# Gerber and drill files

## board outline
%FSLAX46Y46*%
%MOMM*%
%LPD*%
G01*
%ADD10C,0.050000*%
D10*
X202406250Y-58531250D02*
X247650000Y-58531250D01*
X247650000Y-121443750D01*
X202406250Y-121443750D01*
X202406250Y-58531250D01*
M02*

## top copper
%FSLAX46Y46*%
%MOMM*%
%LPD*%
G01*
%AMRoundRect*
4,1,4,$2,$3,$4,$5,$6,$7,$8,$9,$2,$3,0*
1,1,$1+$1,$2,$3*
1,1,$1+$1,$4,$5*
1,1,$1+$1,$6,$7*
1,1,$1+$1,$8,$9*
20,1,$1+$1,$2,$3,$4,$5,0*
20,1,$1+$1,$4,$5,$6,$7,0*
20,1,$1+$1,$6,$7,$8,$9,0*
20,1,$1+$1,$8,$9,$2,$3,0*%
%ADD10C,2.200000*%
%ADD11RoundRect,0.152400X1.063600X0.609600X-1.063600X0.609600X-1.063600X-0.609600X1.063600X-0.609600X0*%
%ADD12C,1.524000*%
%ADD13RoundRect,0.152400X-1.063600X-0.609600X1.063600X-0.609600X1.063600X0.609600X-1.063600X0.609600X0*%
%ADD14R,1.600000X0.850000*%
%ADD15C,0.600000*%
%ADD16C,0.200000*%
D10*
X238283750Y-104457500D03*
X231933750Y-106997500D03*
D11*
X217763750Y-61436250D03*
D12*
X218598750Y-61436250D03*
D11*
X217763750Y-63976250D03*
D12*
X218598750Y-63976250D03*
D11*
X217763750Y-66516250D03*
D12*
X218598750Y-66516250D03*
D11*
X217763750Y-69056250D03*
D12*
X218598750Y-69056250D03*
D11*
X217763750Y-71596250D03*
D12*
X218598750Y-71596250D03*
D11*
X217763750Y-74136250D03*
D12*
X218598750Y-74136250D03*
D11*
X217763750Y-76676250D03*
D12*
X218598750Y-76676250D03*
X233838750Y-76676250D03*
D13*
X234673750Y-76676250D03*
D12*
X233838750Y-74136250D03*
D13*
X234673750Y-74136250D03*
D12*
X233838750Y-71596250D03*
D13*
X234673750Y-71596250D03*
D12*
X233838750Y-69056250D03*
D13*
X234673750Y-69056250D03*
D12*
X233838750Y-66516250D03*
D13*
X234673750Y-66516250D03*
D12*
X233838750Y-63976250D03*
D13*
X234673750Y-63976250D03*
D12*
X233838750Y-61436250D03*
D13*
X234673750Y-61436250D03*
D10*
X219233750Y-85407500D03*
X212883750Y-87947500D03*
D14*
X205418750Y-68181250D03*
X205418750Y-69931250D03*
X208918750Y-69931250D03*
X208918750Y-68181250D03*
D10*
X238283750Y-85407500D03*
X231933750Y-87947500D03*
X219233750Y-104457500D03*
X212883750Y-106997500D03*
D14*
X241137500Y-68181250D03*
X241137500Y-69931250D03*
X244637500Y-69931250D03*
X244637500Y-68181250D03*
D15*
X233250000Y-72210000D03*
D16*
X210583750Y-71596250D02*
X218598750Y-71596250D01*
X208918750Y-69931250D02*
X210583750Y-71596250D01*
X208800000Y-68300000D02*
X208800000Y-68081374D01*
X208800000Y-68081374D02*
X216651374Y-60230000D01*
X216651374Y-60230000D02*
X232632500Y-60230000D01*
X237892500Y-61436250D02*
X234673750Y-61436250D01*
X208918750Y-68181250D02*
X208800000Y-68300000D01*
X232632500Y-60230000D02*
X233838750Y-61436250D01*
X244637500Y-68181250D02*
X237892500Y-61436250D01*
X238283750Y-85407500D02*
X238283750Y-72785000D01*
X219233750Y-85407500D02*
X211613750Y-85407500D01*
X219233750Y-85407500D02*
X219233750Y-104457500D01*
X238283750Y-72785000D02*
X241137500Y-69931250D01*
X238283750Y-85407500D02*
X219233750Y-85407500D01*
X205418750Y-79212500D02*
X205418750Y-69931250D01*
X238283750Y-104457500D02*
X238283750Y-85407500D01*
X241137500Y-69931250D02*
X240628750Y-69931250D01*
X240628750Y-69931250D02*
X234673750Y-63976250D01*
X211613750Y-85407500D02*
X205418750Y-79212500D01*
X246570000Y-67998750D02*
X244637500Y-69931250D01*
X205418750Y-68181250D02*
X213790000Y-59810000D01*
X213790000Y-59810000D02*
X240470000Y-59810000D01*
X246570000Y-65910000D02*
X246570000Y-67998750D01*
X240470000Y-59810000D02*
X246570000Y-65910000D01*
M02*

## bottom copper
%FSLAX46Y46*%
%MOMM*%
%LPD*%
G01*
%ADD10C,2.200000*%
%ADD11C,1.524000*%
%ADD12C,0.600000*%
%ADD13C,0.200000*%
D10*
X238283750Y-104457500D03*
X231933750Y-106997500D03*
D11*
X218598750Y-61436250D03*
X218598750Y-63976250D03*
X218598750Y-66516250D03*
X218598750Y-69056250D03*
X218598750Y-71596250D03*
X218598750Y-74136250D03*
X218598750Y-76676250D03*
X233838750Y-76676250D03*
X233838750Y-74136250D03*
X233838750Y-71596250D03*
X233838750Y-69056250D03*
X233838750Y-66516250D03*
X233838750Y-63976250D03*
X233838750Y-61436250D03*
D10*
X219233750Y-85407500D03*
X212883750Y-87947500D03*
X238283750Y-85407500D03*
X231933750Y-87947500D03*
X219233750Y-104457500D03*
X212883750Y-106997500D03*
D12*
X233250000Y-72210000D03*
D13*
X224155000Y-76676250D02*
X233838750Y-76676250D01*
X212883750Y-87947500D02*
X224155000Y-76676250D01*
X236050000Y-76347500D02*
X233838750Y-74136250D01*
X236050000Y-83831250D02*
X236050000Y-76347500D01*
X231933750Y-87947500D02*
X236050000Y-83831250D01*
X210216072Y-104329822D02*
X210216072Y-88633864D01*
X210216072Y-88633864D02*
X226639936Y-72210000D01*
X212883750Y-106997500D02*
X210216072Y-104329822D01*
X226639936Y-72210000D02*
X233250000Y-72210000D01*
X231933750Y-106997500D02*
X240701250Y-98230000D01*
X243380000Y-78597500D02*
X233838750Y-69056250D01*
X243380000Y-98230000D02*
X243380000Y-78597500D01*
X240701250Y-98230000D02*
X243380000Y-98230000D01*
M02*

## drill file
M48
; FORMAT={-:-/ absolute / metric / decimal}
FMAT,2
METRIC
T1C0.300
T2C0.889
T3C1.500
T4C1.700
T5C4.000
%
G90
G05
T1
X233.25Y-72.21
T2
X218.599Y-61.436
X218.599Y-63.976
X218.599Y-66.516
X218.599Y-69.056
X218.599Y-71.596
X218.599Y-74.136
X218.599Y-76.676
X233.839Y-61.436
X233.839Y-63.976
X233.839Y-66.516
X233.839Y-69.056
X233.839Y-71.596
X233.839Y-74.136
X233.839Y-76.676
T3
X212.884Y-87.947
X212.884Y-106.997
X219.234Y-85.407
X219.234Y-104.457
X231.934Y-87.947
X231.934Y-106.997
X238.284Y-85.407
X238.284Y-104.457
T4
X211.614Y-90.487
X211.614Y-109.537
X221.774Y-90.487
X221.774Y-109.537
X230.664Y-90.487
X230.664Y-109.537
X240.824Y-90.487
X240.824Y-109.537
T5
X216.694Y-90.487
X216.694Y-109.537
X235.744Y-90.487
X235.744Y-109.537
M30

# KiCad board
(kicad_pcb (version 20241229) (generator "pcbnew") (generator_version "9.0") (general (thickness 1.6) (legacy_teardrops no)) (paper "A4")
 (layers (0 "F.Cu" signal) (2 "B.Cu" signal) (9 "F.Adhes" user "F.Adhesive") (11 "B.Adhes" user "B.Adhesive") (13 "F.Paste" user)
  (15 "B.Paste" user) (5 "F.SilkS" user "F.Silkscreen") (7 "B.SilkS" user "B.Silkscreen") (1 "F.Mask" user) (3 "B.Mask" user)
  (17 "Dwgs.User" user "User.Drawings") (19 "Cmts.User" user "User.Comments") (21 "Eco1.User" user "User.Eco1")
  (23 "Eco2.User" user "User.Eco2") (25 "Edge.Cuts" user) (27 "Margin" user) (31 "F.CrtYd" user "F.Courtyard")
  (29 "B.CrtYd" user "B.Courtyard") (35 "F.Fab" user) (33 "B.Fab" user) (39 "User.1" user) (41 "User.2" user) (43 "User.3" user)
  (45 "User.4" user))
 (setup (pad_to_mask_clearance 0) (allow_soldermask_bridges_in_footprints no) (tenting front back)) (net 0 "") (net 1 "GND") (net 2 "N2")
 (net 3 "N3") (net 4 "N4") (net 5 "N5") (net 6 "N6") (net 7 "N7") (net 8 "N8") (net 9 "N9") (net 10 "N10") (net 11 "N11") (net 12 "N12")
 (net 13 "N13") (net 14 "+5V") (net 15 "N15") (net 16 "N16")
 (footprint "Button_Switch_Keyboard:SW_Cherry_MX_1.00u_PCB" (layer "F.Cu") (at 238.28375 104.4575)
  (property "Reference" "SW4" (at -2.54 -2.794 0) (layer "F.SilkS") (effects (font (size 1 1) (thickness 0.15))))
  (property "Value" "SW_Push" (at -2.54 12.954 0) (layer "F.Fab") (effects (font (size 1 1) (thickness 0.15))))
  (pad "" np_thru_hole circle (at -7.62 5.08) (size 1.7 1.7) (drill 1.7) (layers "*.Cu" "*.Mask"))
  (pad "" np_thru_hole circle (at -2.54 5.08) (size 4 4) (drill 4) (layers "*.Cu" "*.Mask"))
  (pad "" np_thru_hole circle (at 2.54 5.08) (size 1.7 1.7) (drill 1.7) (layers "*.Cu" "*.Mask"))
  (pad "1" thru_hole circle (at 0 0) (size 2.2 2.2) (drill 1.5) (layers "*.Cu" "*.Mask") (remove_unused_layers no) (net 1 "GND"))
  (pad "2" thru_hole circle (at -6.35 2.54) (size 2.2 2.2) (drill 1.5) (layers "*.Cu" "*.Mask") (remove_unused_layers no) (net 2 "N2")))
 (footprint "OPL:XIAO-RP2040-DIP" (layer "F.Cu") (at 226.21875 69.05625)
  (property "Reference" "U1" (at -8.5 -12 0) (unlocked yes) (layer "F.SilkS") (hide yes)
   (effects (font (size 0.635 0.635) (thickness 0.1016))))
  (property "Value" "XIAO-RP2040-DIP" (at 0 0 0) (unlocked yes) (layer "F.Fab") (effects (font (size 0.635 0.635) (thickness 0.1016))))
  (pad "1" smd roundrect (at -8.455 -7.62 180) (size 2.432 1.524) (layers "F.Cu" "F.Mask") (roundrect_rratio 0.1) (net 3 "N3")
   (thermal_bridge_angle 45))
  (pad "1" thru_hole circle (at -7.62 -7.62 180) (size 1.524 1.524) (drill 0.889) (layers "*.Cu" "*.Mask") (remove_unused_layers no)
   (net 3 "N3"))
  (pad "2" smd roundrect (at -8.455 -5.08 180) (size 2.432 1.524) (layers "F.Cu" "F.Mask") (roundrect_rratio 0.1) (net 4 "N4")
   (thermal_bridge_angle 45))
  (pad "2" thru_hole circle (at -7.62 -5.08 180) (size 1.524 1.524) (drill 0.889) (layers "*.Cu" "*.Mask") (remove_unused_layers no)
   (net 4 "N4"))
  (pad "3" smd roundrect (at -8.455 -2.54 180) (size 2.432 1.524) (layers "F.Cu" "F.Mask") (roundrect_rratio 0.1) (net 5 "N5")
   (thermal_bridge_angle 45))
  (pad "3" thru_hole circle (at -7.62 -2.54 180) (size 1.524 1.524) (drill 0.889) (layers "*.Cu" "*.Mask") (remove_unused_layers no)
   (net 5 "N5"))
  (pad "4" smd roundrect (at -8.455 0 180) (size 2.432 1.524) (layers "F.Cu" "F.Mask") (roundrect_rratio 0.1) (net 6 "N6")
   (thermal_bridge_angle 45))
  (pad "4" thru_hole circle (at -7.62 0 180) (size 1.524 1.524) (drill 0.889) (layers "*.Cu" "*.Mask") (remove_unused_layers no)
   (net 6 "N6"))
  (pad "5" smd roundrect (at -8.455 2.54 180) (size 2.432 1.524) (layers "F.Cu" "F.Mask") (roundrect_rratio 0.1) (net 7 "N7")
   (thermal_bridge_angle 45))
  (pad "5" thru_hole circle (at -7.62 2.54 180) (size 1.524 1.524) (drill 0.889) (layers "*.Cu" "*.Mask") (remove_unused_layers no)
   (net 7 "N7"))
  (pad "6" smd roundrect (at -8.455 5.08 180) (size 2.432 1.524) (layers "F.Cu" "F.Mask") (roundrect_rratio 0.1) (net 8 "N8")
   (thermal_bridge_angle 45))
  (pad "6" thru_hole circle (at -7.62 5.08 180) (size 1.524 1.524) (drill 0.889) (layers "*.Cu" "*.Mask") (remove_unused_layers no)
   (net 8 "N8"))
  (pad "7" smd roundrect (at -8.455 7.62 180) (size 2.432 1.524) (layers "F.Cu" "F.Mask") (roundrect_rratio 0.1) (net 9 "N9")
   (thermal_bridge_angle 45))
  (pad "7" thru_hole circle (at -7.62 7.62 180) (size 1.524 1.524) (drill 0.889) (layers "*.Cu" "*.Mask") (remove_unused_layers no)
   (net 9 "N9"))
  (pad "8" thru_hole circle (at 7.62 7.62) (size 1.524 1.524) (drill 0.889) (layers "*.Cu" "*.Mask") (remove_unused_layers no)
   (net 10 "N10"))
  (pad "8" smd roundrect (at 8.455 7.62) (size 2.432 1.524) (layers "F.Cu" "F.Mask") (roundrect_rratio 0.1) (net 10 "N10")
   (thermal_bridge_angle 45))
  (pad "9" thru_hole circle (at 7.62 5.08) (size 1.524 1.524) (drill 0.889) (layers "*.Cu" "*.Mask") (remove_unused_layers no)
   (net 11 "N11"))
  (pad "9" smd roundrect (at 8.455 5.08) (size 2.432 1.524) (layers "F.Cu" "F.Mask") (roundrect_rratio 0.1) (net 11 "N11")
   (thermal_bridge_angle 45))
  (pad "10" thru_hole circle (at 7.62 2.54) (size 1.524 1.524) (drill 0.889) (layers "*.Cu" "*.Mask") (remove_unused_layers no)
   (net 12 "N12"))
  (pad "10" smd roundrect (at 8.455 2.54) (size 2.432 1.524) (layers "F.Cu" "F.Mask") (roundrect_rratio 0.1) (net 12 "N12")
   (thermal_bridge_angle 45))
  (pad "11" thru_hole circle (at 7.62 0) (size 1.524 1.524) (drill 0.889) (layers "*.Cu" "*.Mask") (remove_unused_layers no) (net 2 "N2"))
  (pad "11" smd roundrect (at 8.455 0) (size 2.432 1.524) (layers "F.Cu" "F.Mask") (roundrect_rratio 0.1) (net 2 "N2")
   (thermal_bridge_angle 45))
  (pad "12" thru_hole circle (at 7.62 -2.54) (size 1.524 1.524) (drill 0.889) (layers "*.Cu" "*.Mask") (remove_unused_layers no)
   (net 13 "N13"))
  (pad "12" smd roundrect (at 8.455 -2.54) (size 2.432 1.524) (layers "F.Cu" "F.Mask") (roundrect_rratio 0.1) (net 13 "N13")
   (thermal_bridge_angle 45))
  (pad "13" thru_hole circle (at 7.62 -5.08) (size 1.524 1.524) (drill 0.889) (layers "*.Cu" "*.Mask") (remove_unused_layers no)
   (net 1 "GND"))
  (pad "13" smd roundrect (at 8.455 -5.08) (size 2.432 1.524) (layers "F.Cu" "F.Mask") (roundrect_rratio 0.1) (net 1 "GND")
   (thermal_bridge_angle 45))
  (pad "14" thru_hole circle (at 7.62 -7.62) (size 1.524 1.524) (drill 0.889) (layers "*.Cu" "*.Mask") (remove_unused_layers no)
   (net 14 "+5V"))
  (pad "14" smd roundrect (at 8.455 -7.62) (size 2.432 1.524) (layers "F.Cu" "F.Mask") (roundrect_rratio 0.1) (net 14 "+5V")
   (thermal_bridge_angle 45)))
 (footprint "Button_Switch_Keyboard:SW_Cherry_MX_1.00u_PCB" (layer "F.Cu") (at 219.23375 85.4075)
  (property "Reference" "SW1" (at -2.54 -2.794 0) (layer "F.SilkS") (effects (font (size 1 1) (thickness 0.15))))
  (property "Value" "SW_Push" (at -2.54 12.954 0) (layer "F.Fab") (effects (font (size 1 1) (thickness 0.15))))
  (pad "" np_thru_hole circle (at -7.62 5.08) (size 1.7 1.7) (drill 1.7) (layers "*.Cu" "*.Mask"))
  (pad "" np_thru_hole circle (at -2.54 5.08) (size 4 4) (drill 4) (layers "*.Cu" "*.Mask"))
  (pad "" np_thru_hole circle (at 2.54 5.08) (size 1.7 1.7) (drill 1.7) (layers "*.Cu" "*.Mask"))
  (pad "1" thru_hole circle (at 0 0) (size 2.2 2.2) (drill 1.5) (layers "*.Cu" "*.Mask") (remove_unused_layers no) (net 1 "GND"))
  (pad "2" thru_hole circle (at -6.35 2.54) (size 2.2 2.2) (drill 1.5) (layers "*.Cu" "*.Mask") (remove_unused_layers no) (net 10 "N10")))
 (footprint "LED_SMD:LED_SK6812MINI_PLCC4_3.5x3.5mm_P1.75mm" (layer "F.Cu") (at 207.16875 69.05625)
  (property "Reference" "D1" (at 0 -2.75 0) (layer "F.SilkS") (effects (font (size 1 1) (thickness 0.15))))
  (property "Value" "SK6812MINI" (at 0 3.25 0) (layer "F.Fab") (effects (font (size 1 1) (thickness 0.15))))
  (pad "1" smd rect (at -1.75 -0.875) (size 1.6 0.85) (layers "F.Cu" "F.Mask" "F.Paste") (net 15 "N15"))
  (pad "2" smd rect (at -1.75 0.875) (size 1.6 0.85) (layers "F.Cu" "F.Mask" "F.Paste") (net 1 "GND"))
  (pad "3" smd rect (at 1.75 0.875) (size 1.6 0.85) (layers "F.Cu" "F.Mask" "F.Paste") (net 7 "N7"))
  (pad "4" smd rect (at 1.75 -0.875) (size 1.6 0.85) (layers "F.Cu" "F.Mask" "F.Paste") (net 14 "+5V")))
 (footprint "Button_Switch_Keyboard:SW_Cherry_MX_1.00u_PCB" (layer "F.Cu") (at 238.28375 85.4075)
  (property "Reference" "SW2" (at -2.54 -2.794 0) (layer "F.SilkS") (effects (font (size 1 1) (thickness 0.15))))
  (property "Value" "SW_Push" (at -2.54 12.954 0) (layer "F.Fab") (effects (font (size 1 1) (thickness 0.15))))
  (pad "" np_thru_hole circle (at -7.62 5.08) (size 1.7 1.7) (drill 1.7) (layers "*.Cu" "*.Mask"))
  (pad "" np_thru_hole circle (at -2.54 5.08) (size 4 4) (drill 4) (layers "*.Cu" "*.Mask"))
  (pad "" np_thru_hole circle (at 2.54 5.08) (size 1.7 1.7) (drill 1.7) (layers "*.Cu" "*.Mask"))
  (pad "1" thru_hole circle (at 0 0) (size 2.2 2.2) (drill 1.5) (layers "*.Cu" "*.Mask") (remove_unused_layers no) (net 1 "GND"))
  (pad "2" thru_hole circle (at -6.35 2.54) (size 2.2 2.2) (drill 1.5) (layers "*.Cu" "*.Mask") (remove_unused_layers no) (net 11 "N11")))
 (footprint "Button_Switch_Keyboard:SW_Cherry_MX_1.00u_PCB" (layer "F.Cu") (at 219.23375 104.4575)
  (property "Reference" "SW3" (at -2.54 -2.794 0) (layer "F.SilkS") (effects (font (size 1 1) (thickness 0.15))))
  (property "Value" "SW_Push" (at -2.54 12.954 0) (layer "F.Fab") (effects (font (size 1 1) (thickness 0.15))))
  (pad "" np_thru_hole circle (at -7.62 5.08) (size 1.7 1.7) (drill 1.7) (layers "*.Cu" "*.Mask"))
  (pad "" np_thru_hole circle (at -2.54 5.08) (size 4 4) (drill 4) (layers "*.Cu" "*.Mask"))
  (pad "" np_thru_hole circle (at 2.54 5.08) (size 1.7 1.7) (drill 1.7) (layers "*.Cu" "*.Mask"))
  (pad "1" thru_hole circle (at 0 0) (size 2.2 2.2) (drill 1.5) (layers "*.Cu" "*.Mask") (remove_unused_layers no) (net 1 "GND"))
  (pad "2" thru_hole circle (at -6.35 2.54) (size 2.2 2.2) (drill 1.5) (layers "*.Cu" "*.Mask") (remove_unused_layers no) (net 12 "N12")))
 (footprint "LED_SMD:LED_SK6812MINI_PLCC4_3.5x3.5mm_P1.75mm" (layer "F.Cu") (at 242.8875 69.05625)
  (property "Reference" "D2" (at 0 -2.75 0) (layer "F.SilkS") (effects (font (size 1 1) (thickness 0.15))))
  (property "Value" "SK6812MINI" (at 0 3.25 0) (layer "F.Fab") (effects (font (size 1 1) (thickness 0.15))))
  (pad "1" smd rect (at -1.75 -0.875) (size 1.6 0.85) (layers "F.Cu" "F.Mask" "F.Paste") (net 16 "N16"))
  (pad "2" smd rect (at -1.75 0.875) (size 1.6 0.85) (layers "F.Cu" "F.Mask" "F.Paste") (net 1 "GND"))
  (pad "3" smd rect (at 1.75 0.875) (size 1.6 0.85) (layers "F.Cu" "F.Mask" "F.Paste") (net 15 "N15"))
  (pad "4" smd rect (at 1.75 -0.875) (size 1.6 0.85) (layers "F.Cu" "F.Mask" "F.Paste") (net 14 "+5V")))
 (gr_rect (start 202.40625 58.53125) (end 247.65 121.44375) (stroke (width 0.05) (type default)) (fill no) (layer "Edge.Cuts"))
 (segment (start 210.58375 71.59625) (end 218.59875 71.59625) (width 0.2) (layer "F.Cu") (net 7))
 (segment (start 208.91875 69.93125) (end 210.58375 71.59625) (width 0.2) (layer "F.Cu") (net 7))
 (segment (start 208.8 68.3) (end 208.8 68.081374) (width 0.2) (layer "F.Cu") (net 14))
 (segment (start 208.8 68.081374) (end 216.651374 60.23) (width 0.2) (layer "F.Cu") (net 14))
 (segment (start 216.651374 60.23) (end 232.6325 60.23) (width 0.2) (layer "F.Cu") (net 14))
 (segment (start 237.8925 61.43625) (end 234.67375 61.43625) (width 0.2) (layer "F.Cu") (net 14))
 (segment (start 208.91875 68.18125) (end 208.8 68.3) (width 0.2) (layer "F.Cu") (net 14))
 (segment (start 232.6325 60.23) (end 233.83875 61.43625) (width 0.2) (layer "F.Cu") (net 14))
 (segment (start 244.6375 68.18125) (end 237.8925 61.43625) (width 0.2) (layer "F.Cu") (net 14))
 (segment (start 238.28375 85.4075) (end 238.28375 72.785) (width 0.2) (layer "F.Cu") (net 1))
 (segment (start 219.23375 85.4075) (end 211.61375 85.4075) (width 0.2) (layer "F.Cu") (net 1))
 (segment (start 219.23375 85.4075) (end 219.23375 104.4575) (width 0.2) (layer "F.Cu") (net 1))
 (segment (start 238.28375 72.785) (end 241.1375 69.93125) (width 0.2) (layer "F.Cu") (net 1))
 (segment (start 238.28375 85.4075) (end 219.23375 85.4075) (width 0.2) (layer "F.Cu") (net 1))
 (segment (start 205.41875 79.2125) (end 205.41875 69.93125) (width 0.2) (layer "F.Cu") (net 1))
 (segment (start 238.28375 104.4575) (end 238.28375 85.4075) (width 0.2) (layer "F.Cu") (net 1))
 (segment (start 241.1375 69.93125) (end 240.62875 69.93125) (width 0.2) (layer "F.Cu") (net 1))
 (segment (start 240.62875 69.93125) (end 234.67375 63.97625) (width 0.2) (layer "F.Cu") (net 1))
 (segment (start 211.61375 85.4075) (end 205.41875 79.2125) (width 0.2) (layer "F.Cu") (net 1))
 (segment (start 246.57 67.99875) (end 244.6375 69.93125) (width 0.2) (layer "F.Cu") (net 15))
 (segment (start 205.41875 68.18125) (end 213.79 59.81) (width 0.2) (layer "F.Cu") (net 15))
 (segment (start 213.79 59.81) (end 240.47 59.81) (width 0.2) (layer "F.Cu") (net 15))
 (segment (start 246.57 65.91) (end 246.57 67.99875) (width 0.2) (layer "F.Cu") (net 15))
 (segment (start 240.47 59.81) (end 246.57 65.91) (width 0.2) (layer "F.Cu") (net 15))
 (segment (start 224.155 76.67625) (end 233.83875 76.67625) (width 0.2) (layer "B.Cu") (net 10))
 (segment (start 212.88375 87.9475) (end 224.155 76.67625) (width 0.2) (layer "B.Cu") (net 10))
 (segment (start 236.05 76.3475) (end 233.83875 74.13625) (width 0.2) (layer "B.Cu") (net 11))
 (segment (start 236.05 83.83125) (end 236.05 76.3475) (width 0.2) (layer "B.Cu") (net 11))
 (segment (start 231.93375 87.9475) (end 236.05 83.83125) (width 0.2) (layer "B.Cu") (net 11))
 (via (at 233.25 72.21) (size 0.6) (drill 0.3) (layers "F.Cu" "B.Cu") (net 12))
 (segment (start 210.216072 104.329822) (end 210.216072 88.633864) (width 0.2) (layer "B.Cu") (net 12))
 (segment (start 210.216072 88.633864) (end 226.639936 72.21) (width 0.2) (layer "B.Cu") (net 12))
 (segment (start 212.88375 106.9975) (end 210.216072 104.329822) (width 0.2) (layer "B.Cu") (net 12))
 (segment (start 226.639936 72.21) (end 233.25 72.21) (width 0.2) (layer "B.Cu") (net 12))
 (segment (start 231.93375 106.9975) (end 240.70125 98.23) (width 0.2) (layer "B.Cu") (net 2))
 (segment (start 243.38 78.5975) (end 233.83875 69.05625) (width 0.2) (layer "B.Cu") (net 2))
 (segment (start 243.38 98.23) (end 243.38 78.5975) (width 0.2) (layer "B.Cu") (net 2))
 (segment (start 240.70125 98.23) (end 243.38 98.23) (width 0.2) (layer "B.Cu") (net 2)))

